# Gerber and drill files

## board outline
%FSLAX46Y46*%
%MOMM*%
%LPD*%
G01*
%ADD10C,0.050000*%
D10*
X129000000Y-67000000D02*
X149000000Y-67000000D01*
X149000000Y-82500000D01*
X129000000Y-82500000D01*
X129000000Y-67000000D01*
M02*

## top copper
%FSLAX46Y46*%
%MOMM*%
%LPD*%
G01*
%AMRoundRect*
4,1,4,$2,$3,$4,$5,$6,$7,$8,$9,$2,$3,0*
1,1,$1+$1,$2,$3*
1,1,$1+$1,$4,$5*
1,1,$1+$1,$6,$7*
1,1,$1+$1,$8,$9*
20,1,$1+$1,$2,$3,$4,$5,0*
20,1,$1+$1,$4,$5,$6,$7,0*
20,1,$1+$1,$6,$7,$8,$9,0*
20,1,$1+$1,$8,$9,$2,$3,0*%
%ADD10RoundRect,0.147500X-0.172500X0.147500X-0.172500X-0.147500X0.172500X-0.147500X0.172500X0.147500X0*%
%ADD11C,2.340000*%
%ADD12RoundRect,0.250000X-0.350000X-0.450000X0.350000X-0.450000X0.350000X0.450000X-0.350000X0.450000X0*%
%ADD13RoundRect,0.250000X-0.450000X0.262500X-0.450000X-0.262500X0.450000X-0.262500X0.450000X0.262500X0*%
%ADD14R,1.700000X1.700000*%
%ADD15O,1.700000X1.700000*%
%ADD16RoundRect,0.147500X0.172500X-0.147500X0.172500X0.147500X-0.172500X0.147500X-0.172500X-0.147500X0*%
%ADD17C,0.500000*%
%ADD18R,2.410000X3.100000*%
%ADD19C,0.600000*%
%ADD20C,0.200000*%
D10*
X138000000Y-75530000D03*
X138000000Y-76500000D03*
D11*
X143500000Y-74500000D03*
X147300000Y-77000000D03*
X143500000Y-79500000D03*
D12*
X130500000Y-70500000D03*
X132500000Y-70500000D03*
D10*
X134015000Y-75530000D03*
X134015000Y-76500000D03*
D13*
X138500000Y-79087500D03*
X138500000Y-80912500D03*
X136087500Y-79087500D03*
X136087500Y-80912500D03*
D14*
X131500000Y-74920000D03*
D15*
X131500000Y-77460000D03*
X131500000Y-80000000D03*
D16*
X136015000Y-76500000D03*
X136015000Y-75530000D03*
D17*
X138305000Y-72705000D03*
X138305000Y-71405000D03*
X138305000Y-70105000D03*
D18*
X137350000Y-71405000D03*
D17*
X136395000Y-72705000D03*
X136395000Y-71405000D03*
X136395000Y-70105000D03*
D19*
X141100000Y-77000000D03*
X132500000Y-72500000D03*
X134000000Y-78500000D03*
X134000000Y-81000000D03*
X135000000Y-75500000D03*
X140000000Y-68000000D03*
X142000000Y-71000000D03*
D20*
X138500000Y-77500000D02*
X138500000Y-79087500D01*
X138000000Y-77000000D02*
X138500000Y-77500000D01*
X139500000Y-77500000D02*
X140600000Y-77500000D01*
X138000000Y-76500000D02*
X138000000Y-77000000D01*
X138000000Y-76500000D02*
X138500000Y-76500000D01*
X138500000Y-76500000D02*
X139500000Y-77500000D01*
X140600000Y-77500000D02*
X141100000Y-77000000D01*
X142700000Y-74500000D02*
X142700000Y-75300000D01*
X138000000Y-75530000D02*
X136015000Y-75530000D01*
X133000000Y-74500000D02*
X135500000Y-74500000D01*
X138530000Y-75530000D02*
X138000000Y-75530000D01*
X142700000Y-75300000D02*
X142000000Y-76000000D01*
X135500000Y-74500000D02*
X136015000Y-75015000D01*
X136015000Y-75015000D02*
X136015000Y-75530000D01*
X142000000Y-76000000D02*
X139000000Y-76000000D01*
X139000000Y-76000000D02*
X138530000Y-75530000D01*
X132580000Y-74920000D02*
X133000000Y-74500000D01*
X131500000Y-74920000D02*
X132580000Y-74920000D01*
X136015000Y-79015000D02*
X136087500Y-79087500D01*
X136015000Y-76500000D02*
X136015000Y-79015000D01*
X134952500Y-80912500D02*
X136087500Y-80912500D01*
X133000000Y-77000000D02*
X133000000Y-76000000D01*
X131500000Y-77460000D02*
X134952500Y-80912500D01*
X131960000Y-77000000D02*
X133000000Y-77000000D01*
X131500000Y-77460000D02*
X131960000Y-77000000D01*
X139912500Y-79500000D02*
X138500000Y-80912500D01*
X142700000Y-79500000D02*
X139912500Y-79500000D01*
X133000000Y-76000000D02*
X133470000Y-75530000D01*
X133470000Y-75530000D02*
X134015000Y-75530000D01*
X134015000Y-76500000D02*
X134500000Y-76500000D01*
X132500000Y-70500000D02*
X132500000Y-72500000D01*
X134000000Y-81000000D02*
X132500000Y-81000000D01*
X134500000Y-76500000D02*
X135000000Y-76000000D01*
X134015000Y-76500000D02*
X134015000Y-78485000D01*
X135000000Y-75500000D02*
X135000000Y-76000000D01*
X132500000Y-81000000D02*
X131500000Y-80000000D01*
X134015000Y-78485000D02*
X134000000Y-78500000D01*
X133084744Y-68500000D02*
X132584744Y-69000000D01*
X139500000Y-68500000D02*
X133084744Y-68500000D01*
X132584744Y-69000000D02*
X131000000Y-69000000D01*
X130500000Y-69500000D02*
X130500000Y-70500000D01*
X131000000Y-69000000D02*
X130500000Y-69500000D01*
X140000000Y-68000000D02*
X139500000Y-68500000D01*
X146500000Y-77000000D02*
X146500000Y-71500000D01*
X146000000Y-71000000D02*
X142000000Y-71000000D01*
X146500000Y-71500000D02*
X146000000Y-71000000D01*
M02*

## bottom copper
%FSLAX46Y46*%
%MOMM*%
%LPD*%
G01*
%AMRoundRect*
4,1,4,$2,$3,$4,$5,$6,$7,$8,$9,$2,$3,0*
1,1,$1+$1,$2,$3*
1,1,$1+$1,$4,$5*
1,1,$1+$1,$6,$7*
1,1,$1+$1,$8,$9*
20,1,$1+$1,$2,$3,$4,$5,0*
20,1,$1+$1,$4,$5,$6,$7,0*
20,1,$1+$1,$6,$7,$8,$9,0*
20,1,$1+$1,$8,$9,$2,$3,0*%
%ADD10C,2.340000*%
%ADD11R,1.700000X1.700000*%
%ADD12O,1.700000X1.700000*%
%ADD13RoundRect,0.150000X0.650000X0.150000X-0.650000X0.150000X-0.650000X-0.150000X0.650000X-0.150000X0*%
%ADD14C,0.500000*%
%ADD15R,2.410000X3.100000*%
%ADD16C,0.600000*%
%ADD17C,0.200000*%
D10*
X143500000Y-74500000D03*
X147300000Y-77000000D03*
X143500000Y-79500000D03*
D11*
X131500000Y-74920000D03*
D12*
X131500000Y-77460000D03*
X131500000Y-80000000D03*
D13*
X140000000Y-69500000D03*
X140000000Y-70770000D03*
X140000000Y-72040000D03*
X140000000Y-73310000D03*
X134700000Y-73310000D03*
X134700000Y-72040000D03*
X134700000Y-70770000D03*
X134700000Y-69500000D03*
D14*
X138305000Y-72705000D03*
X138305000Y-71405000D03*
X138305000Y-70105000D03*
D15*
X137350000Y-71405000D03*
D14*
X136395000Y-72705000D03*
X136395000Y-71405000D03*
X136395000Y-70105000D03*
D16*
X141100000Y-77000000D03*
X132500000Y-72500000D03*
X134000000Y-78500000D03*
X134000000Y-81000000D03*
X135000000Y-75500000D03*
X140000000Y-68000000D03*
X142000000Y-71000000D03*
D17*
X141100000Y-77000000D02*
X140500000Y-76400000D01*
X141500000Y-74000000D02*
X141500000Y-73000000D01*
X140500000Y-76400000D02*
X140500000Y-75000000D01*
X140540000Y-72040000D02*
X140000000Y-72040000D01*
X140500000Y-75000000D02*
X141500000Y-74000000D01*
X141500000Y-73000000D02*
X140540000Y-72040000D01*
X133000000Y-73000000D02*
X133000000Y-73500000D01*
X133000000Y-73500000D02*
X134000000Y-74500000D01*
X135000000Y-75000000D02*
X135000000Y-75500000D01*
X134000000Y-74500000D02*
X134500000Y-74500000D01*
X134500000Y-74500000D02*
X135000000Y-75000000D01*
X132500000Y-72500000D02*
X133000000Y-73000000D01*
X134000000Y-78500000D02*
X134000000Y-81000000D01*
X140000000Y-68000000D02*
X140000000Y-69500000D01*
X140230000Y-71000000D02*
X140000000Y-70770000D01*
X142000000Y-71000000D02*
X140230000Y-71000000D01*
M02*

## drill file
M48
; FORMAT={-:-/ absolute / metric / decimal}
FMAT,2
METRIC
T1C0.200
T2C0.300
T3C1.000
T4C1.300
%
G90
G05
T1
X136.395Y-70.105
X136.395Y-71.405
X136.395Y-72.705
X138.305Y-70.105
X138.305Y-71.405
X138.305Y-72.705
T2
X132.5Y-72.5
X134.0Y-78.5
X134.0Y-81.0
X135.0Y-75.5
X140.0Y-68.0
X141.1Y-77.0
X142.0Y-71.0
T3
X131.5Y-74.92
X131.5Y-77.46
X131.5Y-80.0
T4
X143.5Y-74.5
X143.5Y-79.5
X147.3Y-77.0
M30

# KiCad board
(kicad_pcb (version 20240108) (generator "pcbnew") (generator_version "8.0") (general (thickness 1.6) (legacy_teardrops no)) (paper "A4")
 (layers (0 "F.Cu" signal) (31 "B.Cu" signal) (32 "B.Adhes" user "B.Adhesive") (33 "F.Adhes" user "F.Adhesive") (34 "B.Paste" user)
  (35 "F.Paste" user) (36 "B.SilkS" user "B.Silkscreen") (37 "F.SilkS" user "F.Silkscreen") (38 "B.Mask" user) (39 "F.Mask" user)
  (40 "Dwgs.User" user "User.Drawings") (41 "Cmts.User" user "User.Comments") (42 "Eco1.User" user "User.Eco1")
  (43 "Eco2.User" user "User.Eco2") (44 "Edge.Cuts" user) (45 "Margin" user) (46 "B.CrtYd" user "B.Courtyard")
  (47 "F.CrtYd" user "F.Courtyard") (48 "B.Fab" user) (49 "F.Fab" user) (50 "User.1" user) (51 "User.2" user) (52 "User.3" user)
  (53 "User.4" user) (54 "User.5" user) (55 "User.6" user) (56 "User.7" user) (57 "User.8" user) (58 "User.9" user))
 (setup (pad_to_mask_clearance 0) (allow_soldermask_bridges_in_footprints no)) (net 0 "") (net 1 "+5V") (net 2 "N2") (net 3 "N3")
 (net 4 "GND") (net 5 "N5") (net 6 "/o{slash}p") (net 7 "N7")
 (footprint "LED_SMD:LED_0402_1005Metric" (layer "F.Cu") (at 138 76.015 -90)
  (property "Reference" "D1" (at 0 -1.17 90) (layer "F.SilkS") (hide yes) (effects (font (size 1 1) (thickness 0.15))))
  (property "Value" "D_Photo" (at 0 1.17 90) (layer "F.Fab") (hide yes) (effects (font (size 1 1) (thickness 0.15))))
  (pad "1" smd roundrect (at -0.485 0 270) (size 0.59 0.64) (layers "F.Cu" "F.Paste" "F.Mask") (roundrect_rratio 0.25) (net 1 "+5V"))
  (pad "2" smd roundrect (at 0.485 0 270) (size 0.59 0.64) (layers "F.Cu" "F.Paste" "F.Mask") (roundrect_rratio 0.25) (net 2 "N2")))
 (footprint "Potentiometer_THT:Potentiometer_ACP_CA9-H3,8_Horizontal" (layer "F.Cu") (at 143.5 74.5)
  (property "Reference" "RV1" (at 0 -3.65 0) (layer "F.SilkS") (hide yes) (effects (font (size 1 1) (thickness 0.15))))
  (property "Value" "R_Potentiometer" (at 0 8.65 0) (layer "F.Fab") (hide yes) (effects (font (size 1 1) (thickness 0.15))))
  (pad "1" thru_hole circle (at 0 0) (size 2.34 2.34) (drill 1.3) (layers "*.Cu" "*.Mask") (remove_unused_layers no) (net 1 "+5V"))
  (pad "2" thru_hole circle (at 3.8 2.5) (size 2.34 2.34) (drill 1.3) (layers "*.Cu" "*.Mask") (remove_unused_layers no) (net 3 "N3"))
  (pad "3" thru_hole circle (at 0 5) (size 2.34 2.34) (drill 1.3) (layers "*.Cu" "*.Mask") (remove_unused_layers no) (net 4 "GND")))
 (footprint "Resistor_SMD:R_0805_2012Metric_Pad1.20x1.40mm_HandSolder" (layer "F.Cu") (at 131.5 70.5)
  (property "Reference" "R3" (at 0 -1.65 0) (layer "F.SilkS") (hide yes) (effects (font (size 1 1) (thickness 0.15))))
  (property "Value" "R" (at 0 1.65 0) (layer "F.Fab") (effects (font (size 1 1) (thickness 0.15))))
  (pad "1" smd roundrect (at -1 0) (size 1.2 1.4) (layers "F.Cu" "F.Paste" "F.Mask") (roundrect_rratio 0.208333) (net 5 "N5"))
  (pad "2" smd roundrect (at 1 0) (size 1.2 1.4) (layers "F.Cu" "F.Paste" "F.Mask") (roundrect_rratio 0.208333) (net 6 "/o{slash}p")))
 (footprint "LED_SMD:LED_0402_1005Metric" (layer "F.Cu") (at 134.015 76.015 -90)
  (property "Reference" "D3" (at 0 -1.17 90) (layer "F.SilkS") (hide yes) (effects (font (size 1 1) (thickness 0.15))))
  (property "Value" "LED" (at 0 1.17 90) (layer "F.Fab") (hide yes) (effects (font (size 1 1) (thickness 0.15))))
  (pad "1" smd roundrect (at -0.485 0 270) (size 0.59 0.64) (layers "F.Cu" "F.Paste" "F.Mask") (roundrect_rratio 0.25) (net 4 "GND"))
  (pad "2" smd roundrect (at 0.485 0 270) (size 0.59 0.64) (layers "F.Cu" "F.Paste" "F.Mask") (roundrect_rratio 0.25) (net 6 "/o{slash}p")))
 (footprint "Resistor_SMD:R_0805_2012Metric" (layer "F.Cu") (at 138.5 80 -90)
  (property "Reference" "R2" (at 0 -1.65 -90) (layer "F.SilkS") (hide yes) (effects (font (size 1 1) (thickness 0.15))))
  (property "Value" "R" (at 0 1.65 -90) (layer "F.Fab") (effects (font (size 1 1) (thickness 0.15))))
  (pad "1" smd roundrect (at -0.9125 0 270) (size 1.025 1.4) (layers "F.Cu" "F.Paste" "F.Mask") (roundrect_rratio 0.243902) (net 2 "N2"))
  (pad "2" smd roundrect (at 0.9125 0 270) (size 1.025 1.4) (layers "F.Cu" "F.Paste" "F.Mask") (roundrect_rratio 0.243902) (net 4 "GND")))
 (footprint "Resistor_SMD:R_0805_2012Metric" (layer "F.Cu") (at 136.0875 80 -90)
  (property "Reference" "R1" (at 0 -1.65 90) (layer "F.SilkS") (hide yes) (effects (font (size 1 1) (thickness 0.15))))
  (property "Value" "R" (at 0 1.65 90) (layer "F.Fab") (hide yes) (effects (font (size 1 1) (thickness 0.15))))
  (pad "1" smd roundrect (at -0.9125 0 270) (size 1.025 1.4) (layers "F.Cu" "F.Paste" "F.Mask") (roundrect_rratio 0.243902) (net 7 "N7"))
  (pad "2" smd roundrect (at 0.9125 0 270) (size 1.025 1.4) (layers "F.Cu" "F.Paste" "F.Mask") (roundrect_rratio 0.243902) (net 4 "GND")))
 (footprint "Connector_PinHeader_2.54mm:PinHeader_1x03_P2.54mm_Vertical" (layer "F.Cu") (at 131.5 74.92)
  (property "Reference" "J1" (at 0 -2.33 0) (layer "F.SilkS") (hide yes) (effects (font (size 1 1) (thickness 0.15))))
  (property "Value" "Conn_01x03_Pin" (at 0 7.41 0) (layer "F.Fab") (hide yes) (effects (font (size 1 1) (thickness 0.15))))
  (pad "1" thru_hole rect (at 0 0) (size 1.7 1.7) (drill 1) (layers "*.Cu" "*.Mask") (remove_unused_layers no) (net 1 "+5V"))
  (pad "2" thru_hole oval (at 0 2.54) (size 1.7 1.7) (drill 1) (layers "*.Cu" "*.Mask") (remove_unused_layers no) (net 4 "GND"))
  (pad "3" thru_hole oval (at 0 5.08) (size 1.7 1.7) (drill 1) (layers "*.Cu" "*.Mask") (remove_unused_layers no) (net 6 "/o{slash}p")))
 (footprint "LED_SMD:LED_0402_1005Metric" (layer "F.Cu") (at 136.015 76.015 90)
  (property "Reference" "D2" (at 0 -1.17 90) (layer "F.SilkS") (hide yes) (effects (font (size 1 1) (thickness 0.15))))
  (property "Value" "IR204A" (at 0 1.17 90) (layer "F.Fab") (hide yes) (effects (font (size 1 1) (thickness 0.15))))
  (pad "1" smd roundrect (at -0.485 0 90) (size 0.59 0.64) (layers "F.Cu" "F.Paste" "F.Mask") (roundrect_rratio 0.25) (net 7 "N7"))
  (pad "2" smd roundrect (at 0.485 0 90) (size 0.59 0.64) (layers "F.Cu" "F.Paste" "F.Mask") (roundrect_rratio 0.25) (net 1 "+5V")))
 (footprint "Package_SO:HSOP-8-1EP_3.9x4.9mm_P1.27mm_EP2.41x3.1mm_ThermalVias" (layer "B.Cu") (at 137.35 71.405 180)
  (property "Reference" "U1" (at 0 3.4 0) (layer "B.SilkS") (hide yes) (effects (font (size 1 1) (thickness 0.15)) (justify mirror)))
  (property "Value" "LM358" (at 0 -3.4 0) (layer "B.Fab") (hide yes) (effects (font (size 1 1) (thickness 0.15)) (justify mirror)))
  (pad "" smd roundrect (at -0.6 -0.775 180) (size 0.97 1.25) (layers "B.Paste") (roundrect_rratio 0.25))
  (pad "" smd roundrect (at -0.6 0.775 180) (size 0.97 1.25) (layers "B.Paste") (roundrect_rratio 0.25))
  (pad "" smd roundrect (at 0.6 -0.775 180) (size 0.97 1.25) (layers "B.Paste") (roundrect_rratio 0.25))
  (pad "" smd roundrect (at 0.6 0.775 180) (size 0.97 1.25) (layers "B.Paste") (roundrect_rratio 0.25))
  (pad "1" smd roundrect (at -2.65 1.905 180) (size 1.6 0.6) (layers "B.Cu" "B.Paste" "B.Mask") (roundrect_rratio 0.25) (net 5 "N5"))
  (pad "2" smd roundrect (at -2.65 0.635 180) (size 1.6 0.6) (layers "B.Cu" "B.Paste" "B.Mask") (roundrect_rratio 0.25) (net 3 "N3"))
  (pad "3" smd roundrect (at -2.65 -0.635 180) (size 1.6 0.6) (layers "B.Cu" "B.Paste" "B.Mask") (roundrect_rratio 0.25) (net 2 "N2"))
  (pad "4" smd roundrect (at -2.65 -1.905 180) (size 1.6 0.6) (layers "B.Cu" "B.Paste" "B.Mask") (roundrect_rratio 0.25))
  (pad "5" smd roundrect (at 2.65 -1.905 180) (size 1.6 0.6) (layers "B.Cu" "B.Paste" "B.Mask") (roundrect_rratio 0.25))
  (pad "6" smd roundrect (at 2.65 -0.635 180) (size 1.6 0.6) (layers "B.Cu" "B.Paste" "B.Mask") (roundrect_rratio 0.25))
  (pad "7" smd roundrect (at 2.65 0.635 180) (size 1.6 0.6) (layers "B.Cu" "B.Paste" "B.Mask") (roundrect_rratio 0.25))
  (pad "8" smd roundrect (at 2.65 1.905 180) (size 1.6 0.6) (layers "B.Cu" "B.Paste" "B.Mask") (roundrect_rratio 0.25))
  (pad "9" thru_hole circle (at -0.955 -1.3 180) (size 0.5 0.5) (drill 0.2) (layers "*.Cu") (remove_unused_layers no))
  (pad "9" thru_hole circle (at -0.955 0 180) (size 0.5 0.5) (drill 0.2) (layers "*.Cu") (remove_unused_layers no))
  (pad "9" thru_hole circle (at -0.955 1.3 180) (size 0.5 0.5) (drill 0.2) (layers "*.Cu") (remove_unused_layers no))
  (pad "9" smd rect (at 0 0 180) (size 2.41 3.1) (layers "F.Cu") (zone_connect 2))
  (pad "9" smd rect (at 0 0 180) (size 2.41 3.1) (layers "B.Cu" "B.Mask") (zone_connect 2))
  (pad "9" thru_hole circle (at 0.955 -1.3 180) (size 0.5 0.5) (drill 0.2) (layers "*.Cu") (remove_unused_layers no))
  (pad "9" thru_hole circle (at 0.955 0 180) (size 0.5 0.5) (drill 0.2) (layers "*.Cu") (remove_unused_layers no))
  (pad "9" thru_hole circle (at 0.955 1.3 180) (size 0.5 0.5) (drill 0.2) (layers "*.Cu") (remove_unused_layers no)))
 (gr_rect (start 129 67) (end 149 82.5) (stroke (width 0.05) (type default)) (fill none) (layer "Edge.Cuts"))
 (segment (start 138.5 77.5) (end 138.5 79.0875) (width 0.2) (layer "F.Cu") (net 2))
 (segment (start 138 77) (end 138.5 77.5) (width 0.2) (layer "F.Cu") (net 2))
 (segment (start 139.5 77.5) (end 140.6 77.5) (width 0.2) (layer "F.Cu") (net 2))
 (segment (start 138 76.5) (end 138 77) (width 0.2) (layer "F.Cu") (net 2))
 (segment (start 138 76.5) (end 138.5 76.5) (width 0.2) (layer "F.Cu") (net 2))
 (segment (start 138.5 76.5) (end 139.5 77.5) (width 0.2) (layer "F.Cu") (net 2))
 (segment (start 140.6 77.5) (end 141.1 77) (width 0.2) (layer "F.Cu") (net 2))
 (via (at 141.1 77) (size 0.6) (drill 0.3) (layers "F.Cu" "B.Cu") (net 2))
 (segment (start 141.1 77) (end 140.5 76.4) (width 0.2) (layer "B.Cu") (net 2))
 (segment (start 141.5 74) (end 141.5 73) (width 0.2) (layer "B.Cu") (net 2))
 (segment (start 140.5 76.4) (end 140.5 75) (width 0.2) (layer "B.Cu") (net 2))
 (segment (start 140.54 72.04) (end 140 72.04) (width 0.2) (layer "B.Cu") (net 2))
 (segment (start 140.5 75) (end 141.5 74) (width 0.2) (layer "B.Cu") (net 2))
 (segment (start 141.5 73) (end 140.54 72.04) (width 0.2) (layer "B.Cu") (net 2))
 (segment (start 142.7 74.5) (end 142.7 75.3) (width 0.2) (layer "F.Cu") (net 1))
 (segment (start 138 75.53) (end 136.015 75.53) (width 0.2) (layer "F.Cu") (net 1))
 (segment (start 133 74.5) (end 135.5 74.5) (width 0.2) (layer "F.Cu") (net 1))
 (segment (start 138.53 75.53) (end 138 75.53) (width 0.2) (layer "F.Cu") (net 1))
 (segment (start 142.7 75.3) (end 142 76) (width 0.2) (layer "F.Cu") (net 1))
 (segment (start 135.5 74.5) (end 136.015 75.015) (width 0.2) (layer "F.Cu") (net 1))
 (segment (start 136.015 75.015) (end 136.015 75.53) (width 0.2) (layer "F.Cu") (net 1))
 (segment (start 142 76) (end 139 76) (width 0.2) (layer "F.Cu") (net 1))
 (segment (start 139 76) (end 138.53 75.53) (width 0.2) (layer "F.Cu") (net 1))
 (segment (start 132.58 74.92) (end 133 74.5) (width 0.2) (layer "F.Cu") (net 1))
 (segment (start 131.5 74.92) (end 132.58 74.92) (width 0.2) (layer "F.Cu") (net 1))
 (segment (start 136.015 79.015) (end 136.0875 79.0875) (width 0.2) (layer "F.Cu") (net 7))
 (segment (start 136.015 76.5) (end 136.015 79.015) (width 0.2) (layer "F.Cu") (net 7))
 (segment (start 134.9525 80.9125) (end 136.0875 80.9125) (width 0.2) (layer "F.Cu") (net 4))
 (segment (start 133 77) (end 133 76) (width 0.2) (layer "F.Cu") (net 4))
 (segment (start 131.5 77.46) (end 134.9525 80.9125) (width 0.2) (layer "F.Cu") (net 4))
 (segment (start 131.96 77) (end 133 77) (width 0.2) (layer "F.Cu") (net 4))
 (segment (start 131.5 77.46) (end 131.96 77) (width 0.2) (layer "F.Cu") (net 4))
 (segment (start 139.9125 79.5) (end 138.5 80.9125) (width 0.2) (layer "F.Cu") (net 4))
 (segment (start 142.7 79.5) (end 139.9125 79.5) (width 0.2) (layer "F.Cu") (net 4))
 (segment (start 133 76) (end 133.47 75.53) (width 0.2) (layer "F.Cu") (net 4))
 (segment (start 133.47 75.53) (end 134.015 75.53) (width 0.2) (layer "F.Cu") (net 4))
 (segment (start 134.015 76.5) (end 134.5 76.5) (width 0.2) (layer "F.Cu") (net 6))
 (segment (start 132.5 70.5) (end 132.5 72.5) (width 0.2) (layer "F.Cu") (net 6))
 (segment (start 134 81) (end 132.5 81) (width 0.2) (layer "F.Cu") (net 6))
 (segment (start 134.5 76.5) (end 135 76) (width 0.2) (layer "F.Cu") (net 6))
 (segment (start 134.015 76.5) (end 134.015 78.485) (width 0.2) (layer "F.Cu") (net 6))
 (segment (start 135 75.5) (end 135 76) (width 0.2) (layer "F.Cu") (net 6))
 (segment (start 132.5 81) (end 131.5 80) (width 0.2) (layer "F.Cu") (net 6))
 (segment (start 134.015 78.485) (end 134 78.5) (width 0.2) (layer "F.Cu") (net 6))
 (via (at 132.5 72.5) (size 0.6) (drill 0.3) (layers "F.Cu" "B.Cu") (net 6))
 (via (at 134 78.5) (size 0.6) (drill 0.3) (layers "F.Cu" "B.Cu") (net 6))
 (via (at 134 81) (size 0.6) (drill 0.3) (layers "F.Cu" "B.Cu") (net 6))
 (via (at 135 75.5) (size 0.6) (drill 0.3) (layers "F.Cu" "B.Cu") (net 6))
 (segment (start 133 73) (end 133 73.5) (width 0.2) (layer "B.Cu") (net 6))
 (segment (start 133 73.5) (end 134 74.5) (width 0.2) (layer "B.Cu") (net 6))
 (segment (start 135 75) (end 135 75.5) (width 0.2) (layer "B.Cu") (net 6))
 (segment (start 134 74.5) (end 134.5 74.5) (width 0.2) (layer "B.Cu") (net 6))
 (segment (start 134.5 74.5) (end 135 75) (width 0.2) (layer "B.Cu") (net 6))
 (segment (start 132.5 72.5) (end 133 73) (width 0.2) (layer "B.Cu") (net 6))
 (segment (start 134 78.5) (end 134 81) (width 0.2) (layer "B.Cu") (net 6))
 (segment (start 133.084744 68.5) (end 132.584744 69) (width 0.2) (layer "F.Cu") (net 5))
 (segment (start 139.5 68.5) (end 133.084744 68.5) (width 0.2) (layer "F.Cu") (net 5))
 (segment (start 132.584744 69) (end 131 69) (width 0.2) (layer "F.Cu") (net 5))
 (segment (start 130.5 69.5) (end 130.5 70.5) (width 0.2) (layer "F.Cu") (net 5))
 (segment (start 131 69) (end 130.5 69.5) (width 0.2) (layer "F.Cu") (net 5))
 (segment (start 140 68) (end 139.5 68.5) (width 0.2) (layer "F.Cu") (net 5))
 (via (at 140 68) (size 0.6) (drill 0.3) (layers "F.Cu" "B.Cu") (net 5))
 (segment (start 140 68) (end 140 69.5) (width 0.2) (layer "B.Cu") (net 5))
 (segment (start 146.5 77) (end 146.5 71.5) (width 0.2) (layer "F.Cu") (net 3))
 (segment (start 146 71) (end 142 71) (width 0.2) (layer "F.Cu") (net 3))
 (segment (start 146.5 71.5) (end 146 71) (width 0.2) (layer "F.Cu") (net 3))
 (via (at 142 71) (size 0.6) (drill 0.3) (layers "F.Cu" "B.Cu") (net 3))
 (segment (start 140.23 71) (end 140 70.77) (width 0.2) (layer "B.Cu") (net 3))
 (segment (start 142 71) (end 140.23 71) (width 0.2) (layer "B.Cu") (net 3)))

